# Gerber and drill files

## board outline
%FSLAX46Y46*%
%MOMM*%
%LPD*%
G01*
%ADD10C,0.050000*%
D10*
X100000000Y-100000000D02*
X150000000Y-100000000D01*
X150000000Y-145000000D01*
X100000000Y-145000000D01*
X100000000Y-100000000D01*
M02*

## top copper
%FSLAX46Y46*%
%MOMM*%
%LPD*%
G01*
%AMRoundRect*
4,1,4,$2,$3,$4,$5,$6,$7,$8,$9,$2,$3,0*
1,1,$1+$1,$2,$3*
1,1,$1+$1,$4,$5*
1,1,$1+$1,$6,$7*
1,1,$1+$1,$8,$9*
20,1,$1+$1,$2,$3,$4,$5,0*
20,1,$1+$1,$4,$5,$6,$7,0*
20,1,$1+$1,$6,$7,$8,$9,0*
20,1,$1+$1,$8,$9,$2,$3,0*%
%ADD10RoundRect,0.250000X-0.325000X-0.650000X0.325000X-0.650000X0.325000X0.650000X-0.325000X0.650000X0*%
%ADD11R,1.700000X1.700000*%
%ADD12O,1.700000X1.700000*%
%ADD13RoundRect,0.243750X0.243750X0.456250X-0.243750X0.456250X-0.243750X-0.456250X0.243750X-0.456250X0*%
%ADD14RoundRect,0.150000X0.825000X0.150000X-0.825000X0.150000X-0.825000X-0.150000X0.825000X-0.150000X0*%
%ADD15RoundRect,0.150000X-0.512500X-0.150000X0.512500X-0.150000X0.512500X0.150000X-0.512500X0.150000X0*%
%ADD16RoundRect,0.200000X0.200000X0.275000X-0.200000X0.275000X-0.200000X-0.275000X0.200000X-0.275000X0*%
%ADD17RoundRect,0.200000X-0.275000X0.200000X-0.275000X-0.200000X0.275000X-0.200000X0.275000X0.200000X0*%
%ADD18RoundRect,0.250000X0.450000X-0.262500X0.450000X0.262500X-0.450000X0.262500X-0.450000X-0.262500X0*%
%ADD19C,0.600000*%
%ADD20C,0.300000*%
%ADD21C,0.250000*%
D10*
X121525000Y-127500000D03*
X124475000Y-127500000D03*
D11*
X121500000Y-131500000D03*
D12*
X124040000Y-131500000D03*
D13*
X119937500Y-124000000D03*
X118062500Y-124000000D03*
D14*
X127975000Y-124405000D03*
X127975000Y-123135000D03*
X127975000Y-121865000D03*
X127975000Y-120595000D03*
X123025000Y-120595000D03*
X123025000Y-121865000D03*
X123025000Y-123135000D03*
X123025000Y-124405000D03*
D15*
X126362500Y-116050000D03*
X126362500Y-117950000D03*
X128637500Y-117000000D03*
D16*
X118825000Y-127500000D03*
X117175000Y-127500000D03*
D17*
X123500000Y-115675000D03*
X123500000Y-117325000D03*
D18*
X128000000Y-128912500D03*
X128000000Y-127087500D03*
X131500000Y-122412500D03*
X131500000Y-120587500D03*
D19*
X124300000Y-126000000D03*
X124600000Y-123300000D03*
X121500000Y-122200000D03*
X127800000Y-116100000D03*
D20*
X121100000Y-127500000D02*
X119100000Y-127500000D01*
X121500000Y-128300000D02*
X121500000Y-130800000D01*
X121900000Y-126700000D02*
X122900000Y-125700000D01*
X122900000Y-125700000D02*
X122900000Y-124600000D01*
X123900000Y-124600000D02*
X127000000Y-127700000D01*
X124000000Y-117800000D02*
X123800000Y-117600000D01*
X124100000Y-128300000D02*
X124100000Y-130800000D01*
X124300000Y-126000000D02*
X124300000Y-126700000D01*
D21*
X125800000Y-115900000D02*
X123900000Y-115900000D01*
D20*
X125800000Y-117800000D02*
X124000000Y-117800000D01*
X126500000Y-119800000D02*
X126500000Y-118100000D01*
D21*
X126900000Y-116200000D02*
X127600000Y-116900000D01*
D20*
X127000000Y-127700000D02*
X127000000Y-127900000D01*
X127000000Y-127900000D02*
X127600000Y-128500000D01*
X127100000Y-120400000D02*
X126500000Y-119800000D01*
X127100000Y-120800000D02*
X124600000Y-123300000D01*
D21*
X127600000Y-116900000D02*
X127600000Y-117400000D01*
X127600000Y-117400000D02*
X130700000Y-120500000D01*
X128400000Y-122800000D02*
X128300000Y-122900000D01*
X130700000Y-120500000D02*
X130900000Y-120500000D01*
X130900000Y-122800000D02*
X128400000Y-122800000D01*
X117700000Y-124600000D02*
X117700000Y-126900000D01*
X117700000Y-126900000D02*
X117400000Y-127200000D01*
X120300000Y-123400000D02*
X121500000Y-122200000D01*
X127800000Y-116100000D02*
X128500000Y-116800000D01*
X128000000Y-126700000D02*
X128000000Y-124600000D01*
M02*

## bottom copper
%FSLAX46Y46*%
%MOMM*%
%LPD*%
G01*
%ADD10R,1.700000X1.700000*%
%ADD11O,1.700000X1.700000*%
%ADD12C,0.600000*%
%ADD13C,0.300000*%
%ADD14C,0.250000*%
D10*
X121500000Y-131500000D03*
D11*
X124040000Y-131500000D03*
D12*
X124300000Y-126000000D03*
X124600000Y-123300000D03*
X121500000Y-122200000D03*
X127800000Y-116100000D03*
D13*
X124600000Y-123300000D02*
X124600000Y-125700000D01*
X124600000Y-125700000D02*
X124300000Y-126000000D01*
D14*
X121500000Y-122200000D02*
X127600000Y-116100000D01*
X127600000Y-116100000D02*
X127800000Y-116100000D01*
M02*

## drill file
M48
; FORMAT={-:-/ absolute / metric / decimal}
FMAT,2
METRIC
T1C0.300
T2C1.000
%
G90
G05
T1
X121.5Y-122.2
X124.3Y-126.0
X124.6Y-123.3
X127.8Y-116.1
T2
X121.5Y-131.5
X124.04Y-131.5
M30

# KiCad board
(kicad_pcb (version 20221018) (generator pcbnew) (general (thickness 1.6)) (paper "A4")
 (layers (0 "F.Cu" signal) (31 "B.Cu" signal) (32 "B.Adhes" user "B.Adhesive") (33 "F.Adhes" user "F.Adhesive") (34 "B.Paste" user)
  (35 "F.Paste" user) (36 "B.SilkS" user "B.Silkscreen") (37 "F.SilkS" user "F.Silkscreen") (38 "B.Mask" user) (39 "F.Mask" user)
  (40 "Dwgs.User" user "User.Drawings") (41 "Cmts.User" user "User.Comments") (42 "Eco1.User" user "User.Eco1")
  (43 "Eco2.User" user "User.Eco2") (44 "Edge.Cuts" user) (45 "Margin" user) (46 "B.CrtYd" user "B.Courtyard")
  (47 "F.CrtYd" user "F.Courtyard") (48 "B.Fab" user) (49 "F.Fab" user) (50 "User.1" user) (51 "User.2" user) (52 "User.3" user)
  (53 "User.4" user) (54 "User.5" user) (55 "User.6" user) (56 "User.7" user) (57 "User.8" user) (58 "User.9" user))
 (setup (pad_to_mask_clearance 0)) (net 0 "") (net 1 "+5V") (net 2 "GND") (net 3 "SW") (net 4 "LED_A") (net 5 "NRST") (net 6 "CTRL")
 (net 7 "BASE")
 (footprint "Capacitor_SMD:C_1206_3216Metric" (layer "F.Cu") (at 123 127.5)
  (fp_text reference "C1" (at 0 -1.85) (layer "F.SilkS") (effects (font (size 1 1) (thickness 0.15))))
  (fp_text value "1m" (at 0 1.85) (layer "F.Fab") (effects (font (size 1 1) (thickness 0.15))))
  (pad "1" smd roundrect (at -1.475 0) (size 1.15 1.8) (layers "F.Cu" "F.Paste" "F.Mask") (roundrect_rratio 0.217391) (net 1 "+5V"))
  (pad "2" smd roundrect (at 1.475 0) (size 1.15 1.8) (layers "F.Cu" "F.Paste" "F.Mask") (roundrect_rratio 0.217391) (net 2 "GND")))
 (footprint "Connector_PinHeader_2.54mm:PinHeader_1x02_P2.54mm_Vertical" (layer "F.Cu") (at 121.5 131.5 90)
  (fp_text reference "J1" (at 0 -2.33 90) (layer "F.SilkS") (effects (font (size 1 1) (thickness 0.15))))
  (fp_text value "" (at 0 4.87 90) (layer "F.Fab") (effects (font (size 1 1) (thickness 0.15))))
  (pad "1" thru_hole rect (at 0 0 90) (size 1.7 1.7) (drill 1) (layers "*.Cu" "*.Mask") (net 1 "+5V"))
  (pad "2" thru_hole oval (at 0 2.54 90) (size 1.7 1.7) (drill 1) (layers "*.Cu" "*.Mask") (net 2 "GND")))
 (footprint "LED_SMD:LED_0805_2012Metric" (layer "F.Cu") (at 119 124 180)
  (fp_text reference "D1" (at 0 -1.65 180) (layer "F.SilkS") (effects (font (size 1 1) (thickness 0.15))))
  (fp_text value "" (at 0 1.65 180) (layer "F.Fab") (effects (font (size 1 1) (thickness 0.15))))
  (pad "1" smd roundrect (at -0.9375 0 180) (size 0.975 1.4) (layers "F.Cu" "F.Paste" "F.Mask") (roundrect_rratio 0.25) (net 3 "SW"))
  (pad "2" smd roundrect (at 0.9375 0 180) (size 0.975 1.4) (layers "F.Cu" "F.Paste" "F.Mask") (roundrect_rratio 0.25) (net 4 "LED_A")))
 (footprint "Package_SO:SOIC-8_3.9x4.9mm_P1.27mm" (layer "F.Cu") (at 125.5 122.5 180)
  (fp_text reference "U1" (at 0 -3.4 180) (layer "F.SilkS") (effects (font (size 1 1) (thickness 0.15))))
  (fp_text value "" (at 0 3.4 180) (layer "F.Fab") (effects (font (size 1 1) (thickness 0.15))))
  (pad "1" smd roundrect (at -2.475 -1.905 180) (size 1.95 0.6) (layers "F.Cu" "F.Paste" "F.Mask") (roundrect_rratio 0.25) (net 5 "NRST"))
  (pad "2" smd roundrect (at -2.475 -0.635 180) (size 1.95 0.6) (layers "F.Cu" "F.Paste" "F.Mask") (roundrect_rratio 0.25) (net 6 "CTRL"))
  (pad "3" smd roundrect (at -2.475 0.635 180) (size 1.95 0.6) (layers "F.Cu" "F.Paste" "F.Mask") (roundrect_rratio 0.25))
  (pad "4" smd roundrect (at -2.475 1.905 180) (size 1.95 0.6) (layers "F.Cu" "F.Paste" "F.Mask") (roundrect_rratio 0.25) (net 2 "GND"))
  (pad "5" smd roundrect (at 2.475 1.905 180) (size 1.95 0.6) (layers "F.Cu" "F.Paste" "F.Mask") (roundrect_rratio 0.25))
  (pad "6" smd roundrect (at 2.475 0.635 180) (size 1.95 0.6) (layers "F.Cu" "F.Paste" "F.Mask") (roundrect_rratio 0.25))
  (pad "7" smd roundrect (at 2.475 -0.635 180) (size 1.95 0.6) (layers "F.Cu" "F.Paste" "F.Mask") (roundrect_rratio 0.25))
  (pad "8" smd roundrect (at 2.475 -1.905 180) (size 1.95 0.6) (layers "F.Cu" "F.Paste" "F.Mask") (roundrect_rratio 0.25) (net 1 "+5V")))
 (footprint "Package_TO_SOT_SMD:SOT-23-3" (layer "F.Cu") (at 127.5 117)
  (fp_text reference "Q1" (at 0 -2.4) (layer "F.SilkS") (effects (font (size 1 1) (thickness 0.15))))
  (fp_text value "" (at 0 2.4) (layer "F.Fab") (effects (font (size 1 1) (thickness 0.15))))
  (pad "1" smd roundrect (at -1.1375 -0.95) (size 1.325 0.6) (layers "F.Cu" "F.Paste" "F.Mask") (roundrect_rratio 0.25) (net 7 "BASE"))
  (pad "2" smd roundrect (at -1.1375 0.95) (size 1.325 0.6) (layers "F.Cu" "F.Paste" "F.Mask") (roundrect_rratio 0.25) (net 2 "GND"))
  (pad "3" smd roundrect (at 1.1375 0) (size 1.325 0.6) (layers "F.Cu" "F.Paste" "F.Mask") (roundrect_rratio 0.25) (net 3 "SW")))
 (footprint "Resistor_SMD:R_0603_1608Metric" (layer "F.Cu") (at 118 127.5 180)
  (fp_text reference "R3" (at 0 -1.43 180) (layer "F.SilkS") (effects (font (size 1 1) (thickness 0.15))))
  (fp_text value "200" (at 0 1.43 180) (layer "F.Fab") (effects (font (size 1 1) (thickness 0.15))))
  (pad "1" smd roundrect (at -0.825 0 180) (size 0.8 0.95) (layers "F.Cu" "F.Paste" "F.Mask") (roundrect_rratio 0.25) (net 1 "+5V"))
  (pad "2" smd roundrect (at 0.825 0 180) (size 0.8 0.95) (layers "F.Cu" "F.Paste" "F.Mask") (roundrect_rratio 0.25) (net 4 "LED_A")))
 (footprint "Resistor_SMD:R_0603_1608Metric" (layer "F.Cu") (at 123.5 116.5 -90)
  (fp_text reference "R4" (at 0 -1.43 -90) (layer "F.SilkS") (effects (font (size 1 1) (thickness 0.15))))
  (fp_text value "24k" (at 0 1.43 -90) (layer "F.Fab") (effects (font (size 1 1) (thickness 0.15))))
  (pad "1" smd roundrect (at -0.825 0 270) (size 0.8 0.95) (layers "F.Cu" "F.Paste" "F.Mask") (roundrect_rratio 0.25) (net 7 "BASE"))
  (pad "2" smd roundrect (at 0.825 0 270) (size 0.8 0.95) (layers "F.Cu" "F.Paste" "F.Mask") (roundrect_rratio 0.25) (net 2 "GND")))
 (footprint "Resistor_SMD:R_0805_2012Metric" (layer "F.Cu") (at 128 128 90)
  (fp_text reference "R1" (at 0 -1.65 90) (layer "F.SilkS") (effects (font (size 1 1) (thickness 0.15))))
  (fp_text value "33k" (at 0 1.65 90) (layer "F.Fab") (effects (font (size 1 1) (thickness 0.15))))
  (pad "1" smd roundrect (at -0.9125 0 90) (size 1.025 1.4) (layers "F.Cu" "F.Paste" "F.Mask") (roundrect_rratio 0.243902) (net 1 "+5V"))
  (pad "2" smd roundrect (at 0.9125 0 90) (size 1.025 1.4) (layers "F.Cu" "F.Paste" "F.Mask") (roundrect_rratio 0.243902) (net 5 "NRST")))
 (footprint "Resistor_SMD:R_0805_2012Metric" (layer "F.Cu") (at 131.5 121.5 90)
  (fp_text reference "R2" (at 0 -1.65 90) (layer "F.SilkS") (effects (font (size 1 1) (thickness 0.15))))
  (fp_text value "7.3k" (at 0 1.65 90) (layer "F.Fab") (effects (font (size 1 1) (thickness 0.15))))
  (pad "1" smd roundrect (at -0.9125 0 90) (size 1.025 1.4) (layers "F.Cu" "F.Paste" "F.Mask") (roundrect_rratio 0.243902) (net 6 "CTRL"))
  (pad "2" smd roundrect (at 0.9125 0 90) (size 1.025 1.4) (layers "F.Cu" "F.Paste" "F.Mask") (roundrect_rratio 0.243902) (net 7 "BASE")))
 (gr_rect (start 100 100) (end 150 145) (stroke (width 0.05) (type default)) (fill none) (layer "Edge.Cuts"))
 (segment (start 121.1 127.5) (end 119.1 127.5) (width 0.3) (layer "F.Cu") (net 1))
 (segment (start 121.5 128.3) (end 121.5 130.8) (width 0.3) (layer "F.Cu") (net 1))
 (segment (start 121.9 126.7) (end 122.9 125.7) (width 0.3) (layer "F.Cu") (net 1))
 (segment (start 122.9 125.7) (end 122.9 124.6) (width 0.3) (layer "F.Cu") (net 1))
 (segment (start 123.9 124.6) (end 127 127.7) (width 0.3) (layer "F.Cu") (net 1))
 (segment (start 124 117.8) (end 123.8 117.6) (width 0.3) (layer "F.Cu") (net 2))
 (segment (start 124.1 128.3) (end 124.1 130.8) (width 0.3) (layer "F.Cu") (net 2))
 (segment (start 124.3 126) (end 124.3 126.7) (width 0.3) (layer "F.Cu") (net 2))
 (segment (start 125.8 115.9) (end 123.9 115.9) (width 0.25) (layer "F.Cu") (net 7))
 (segment (start 125.8 117.8) (end 124 117.8) (width 0.3) (layer "F.Cu") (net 2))
 (segment (start 126.5 119.8) (end 126.5 118.1) (width 0.3) (layer "F.Cu") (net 2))
 (segment (start 126.9 116.2) (end 127.6 116.9) (width 0.25) (layer "F.Cu") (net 7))
 (segment (start 127 127.7) (end 127 127.9) (width 0.3) (layer "F.Cu") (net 1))
 (segment (start 127 127.9) (end 127.6 128.5) (width 0.3) (layer "F.Cu") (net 1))
 (segment (start 127.1 120.4) (end 126.5 119.8) (width 0.3) (layer "F.Cu") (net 2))
 (segment (start 127.1 120.8) (end 124.6 123.3) (width 0.3) (layer "F.Cu") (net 2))
 (segment (start 127.6 116.9) (end 127.6 117.4) (width 0.25) (layer "F.Cu") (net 7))
 (segment (start 127.6 117.4) (end 130.7 120.5) (width 0.25) (layer "F.Cu") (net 7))
 (segment (start 128.4 122.8) (end 128.3 122.9) (width 0.25) (layer "F.Cu") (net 6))
 (segment (start 130.7 120.5) (end 130.9 120.5) (width 0.25) (layer "F.Cu") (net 7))
 (segment (start 130.9 122.8) (end 128.4 122.8) (width 0.25) (layer "F.Cu") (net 6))
 (via (at 124.3 126) (size 0.6) (drill 0.3) (layers "F.Cu" "B.Cu") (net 2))
 (via (at 124.6 123.3) (size 0.6) (drill 0.3) (layers "F.Cu" "B.Cu") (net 2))
 (segment (start 117.7 124.6) (end 117.7 126.9) (width 0.25) (layer "F.Cu") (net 4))
 (segment (start 117.7 126.9) (end 117.4 127.2) (width 0.25) (layer "F.Cu") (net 4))
 (segment (start 120.3 123.4) (end 121.5 122.2) (width 0.25) (layer "F.Cu") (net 3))
 (segment (start 124.6 123.3) (end 124.6 125.7) (width 0.3) (layer "B.Cu") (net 2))
 (segment (start 124.6 125.7) (end 124.3 126) (width 0.3) (layer "B.Cu") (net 2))
 (segment (start 127.8 116.1) (end 128.5 116.8) (width 0.25) (layer "F.Cu") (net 3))
 (segment (start 128 126.7) (end 128 124.6) (width 0.25) (layer "F.Cu") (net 5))
 (via (at 121.5 122.2) (size 0.6) (drill 0.3) (layers "F.Cu" "B.Cu") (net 3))
 (via (at 127.8 116.1) (size 0.6) (drill 0.3) (layers "F.Cu" "B.Cu") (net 3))
 (segment (start 121.5 122.2) (end 127.6 116.1) (width 0.25) (layer "B.Cu") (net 3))
 (segment (start 127.6 116.1) (end 127.8 116.1) (width 0.25) (layer "B.Cu") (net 3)))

